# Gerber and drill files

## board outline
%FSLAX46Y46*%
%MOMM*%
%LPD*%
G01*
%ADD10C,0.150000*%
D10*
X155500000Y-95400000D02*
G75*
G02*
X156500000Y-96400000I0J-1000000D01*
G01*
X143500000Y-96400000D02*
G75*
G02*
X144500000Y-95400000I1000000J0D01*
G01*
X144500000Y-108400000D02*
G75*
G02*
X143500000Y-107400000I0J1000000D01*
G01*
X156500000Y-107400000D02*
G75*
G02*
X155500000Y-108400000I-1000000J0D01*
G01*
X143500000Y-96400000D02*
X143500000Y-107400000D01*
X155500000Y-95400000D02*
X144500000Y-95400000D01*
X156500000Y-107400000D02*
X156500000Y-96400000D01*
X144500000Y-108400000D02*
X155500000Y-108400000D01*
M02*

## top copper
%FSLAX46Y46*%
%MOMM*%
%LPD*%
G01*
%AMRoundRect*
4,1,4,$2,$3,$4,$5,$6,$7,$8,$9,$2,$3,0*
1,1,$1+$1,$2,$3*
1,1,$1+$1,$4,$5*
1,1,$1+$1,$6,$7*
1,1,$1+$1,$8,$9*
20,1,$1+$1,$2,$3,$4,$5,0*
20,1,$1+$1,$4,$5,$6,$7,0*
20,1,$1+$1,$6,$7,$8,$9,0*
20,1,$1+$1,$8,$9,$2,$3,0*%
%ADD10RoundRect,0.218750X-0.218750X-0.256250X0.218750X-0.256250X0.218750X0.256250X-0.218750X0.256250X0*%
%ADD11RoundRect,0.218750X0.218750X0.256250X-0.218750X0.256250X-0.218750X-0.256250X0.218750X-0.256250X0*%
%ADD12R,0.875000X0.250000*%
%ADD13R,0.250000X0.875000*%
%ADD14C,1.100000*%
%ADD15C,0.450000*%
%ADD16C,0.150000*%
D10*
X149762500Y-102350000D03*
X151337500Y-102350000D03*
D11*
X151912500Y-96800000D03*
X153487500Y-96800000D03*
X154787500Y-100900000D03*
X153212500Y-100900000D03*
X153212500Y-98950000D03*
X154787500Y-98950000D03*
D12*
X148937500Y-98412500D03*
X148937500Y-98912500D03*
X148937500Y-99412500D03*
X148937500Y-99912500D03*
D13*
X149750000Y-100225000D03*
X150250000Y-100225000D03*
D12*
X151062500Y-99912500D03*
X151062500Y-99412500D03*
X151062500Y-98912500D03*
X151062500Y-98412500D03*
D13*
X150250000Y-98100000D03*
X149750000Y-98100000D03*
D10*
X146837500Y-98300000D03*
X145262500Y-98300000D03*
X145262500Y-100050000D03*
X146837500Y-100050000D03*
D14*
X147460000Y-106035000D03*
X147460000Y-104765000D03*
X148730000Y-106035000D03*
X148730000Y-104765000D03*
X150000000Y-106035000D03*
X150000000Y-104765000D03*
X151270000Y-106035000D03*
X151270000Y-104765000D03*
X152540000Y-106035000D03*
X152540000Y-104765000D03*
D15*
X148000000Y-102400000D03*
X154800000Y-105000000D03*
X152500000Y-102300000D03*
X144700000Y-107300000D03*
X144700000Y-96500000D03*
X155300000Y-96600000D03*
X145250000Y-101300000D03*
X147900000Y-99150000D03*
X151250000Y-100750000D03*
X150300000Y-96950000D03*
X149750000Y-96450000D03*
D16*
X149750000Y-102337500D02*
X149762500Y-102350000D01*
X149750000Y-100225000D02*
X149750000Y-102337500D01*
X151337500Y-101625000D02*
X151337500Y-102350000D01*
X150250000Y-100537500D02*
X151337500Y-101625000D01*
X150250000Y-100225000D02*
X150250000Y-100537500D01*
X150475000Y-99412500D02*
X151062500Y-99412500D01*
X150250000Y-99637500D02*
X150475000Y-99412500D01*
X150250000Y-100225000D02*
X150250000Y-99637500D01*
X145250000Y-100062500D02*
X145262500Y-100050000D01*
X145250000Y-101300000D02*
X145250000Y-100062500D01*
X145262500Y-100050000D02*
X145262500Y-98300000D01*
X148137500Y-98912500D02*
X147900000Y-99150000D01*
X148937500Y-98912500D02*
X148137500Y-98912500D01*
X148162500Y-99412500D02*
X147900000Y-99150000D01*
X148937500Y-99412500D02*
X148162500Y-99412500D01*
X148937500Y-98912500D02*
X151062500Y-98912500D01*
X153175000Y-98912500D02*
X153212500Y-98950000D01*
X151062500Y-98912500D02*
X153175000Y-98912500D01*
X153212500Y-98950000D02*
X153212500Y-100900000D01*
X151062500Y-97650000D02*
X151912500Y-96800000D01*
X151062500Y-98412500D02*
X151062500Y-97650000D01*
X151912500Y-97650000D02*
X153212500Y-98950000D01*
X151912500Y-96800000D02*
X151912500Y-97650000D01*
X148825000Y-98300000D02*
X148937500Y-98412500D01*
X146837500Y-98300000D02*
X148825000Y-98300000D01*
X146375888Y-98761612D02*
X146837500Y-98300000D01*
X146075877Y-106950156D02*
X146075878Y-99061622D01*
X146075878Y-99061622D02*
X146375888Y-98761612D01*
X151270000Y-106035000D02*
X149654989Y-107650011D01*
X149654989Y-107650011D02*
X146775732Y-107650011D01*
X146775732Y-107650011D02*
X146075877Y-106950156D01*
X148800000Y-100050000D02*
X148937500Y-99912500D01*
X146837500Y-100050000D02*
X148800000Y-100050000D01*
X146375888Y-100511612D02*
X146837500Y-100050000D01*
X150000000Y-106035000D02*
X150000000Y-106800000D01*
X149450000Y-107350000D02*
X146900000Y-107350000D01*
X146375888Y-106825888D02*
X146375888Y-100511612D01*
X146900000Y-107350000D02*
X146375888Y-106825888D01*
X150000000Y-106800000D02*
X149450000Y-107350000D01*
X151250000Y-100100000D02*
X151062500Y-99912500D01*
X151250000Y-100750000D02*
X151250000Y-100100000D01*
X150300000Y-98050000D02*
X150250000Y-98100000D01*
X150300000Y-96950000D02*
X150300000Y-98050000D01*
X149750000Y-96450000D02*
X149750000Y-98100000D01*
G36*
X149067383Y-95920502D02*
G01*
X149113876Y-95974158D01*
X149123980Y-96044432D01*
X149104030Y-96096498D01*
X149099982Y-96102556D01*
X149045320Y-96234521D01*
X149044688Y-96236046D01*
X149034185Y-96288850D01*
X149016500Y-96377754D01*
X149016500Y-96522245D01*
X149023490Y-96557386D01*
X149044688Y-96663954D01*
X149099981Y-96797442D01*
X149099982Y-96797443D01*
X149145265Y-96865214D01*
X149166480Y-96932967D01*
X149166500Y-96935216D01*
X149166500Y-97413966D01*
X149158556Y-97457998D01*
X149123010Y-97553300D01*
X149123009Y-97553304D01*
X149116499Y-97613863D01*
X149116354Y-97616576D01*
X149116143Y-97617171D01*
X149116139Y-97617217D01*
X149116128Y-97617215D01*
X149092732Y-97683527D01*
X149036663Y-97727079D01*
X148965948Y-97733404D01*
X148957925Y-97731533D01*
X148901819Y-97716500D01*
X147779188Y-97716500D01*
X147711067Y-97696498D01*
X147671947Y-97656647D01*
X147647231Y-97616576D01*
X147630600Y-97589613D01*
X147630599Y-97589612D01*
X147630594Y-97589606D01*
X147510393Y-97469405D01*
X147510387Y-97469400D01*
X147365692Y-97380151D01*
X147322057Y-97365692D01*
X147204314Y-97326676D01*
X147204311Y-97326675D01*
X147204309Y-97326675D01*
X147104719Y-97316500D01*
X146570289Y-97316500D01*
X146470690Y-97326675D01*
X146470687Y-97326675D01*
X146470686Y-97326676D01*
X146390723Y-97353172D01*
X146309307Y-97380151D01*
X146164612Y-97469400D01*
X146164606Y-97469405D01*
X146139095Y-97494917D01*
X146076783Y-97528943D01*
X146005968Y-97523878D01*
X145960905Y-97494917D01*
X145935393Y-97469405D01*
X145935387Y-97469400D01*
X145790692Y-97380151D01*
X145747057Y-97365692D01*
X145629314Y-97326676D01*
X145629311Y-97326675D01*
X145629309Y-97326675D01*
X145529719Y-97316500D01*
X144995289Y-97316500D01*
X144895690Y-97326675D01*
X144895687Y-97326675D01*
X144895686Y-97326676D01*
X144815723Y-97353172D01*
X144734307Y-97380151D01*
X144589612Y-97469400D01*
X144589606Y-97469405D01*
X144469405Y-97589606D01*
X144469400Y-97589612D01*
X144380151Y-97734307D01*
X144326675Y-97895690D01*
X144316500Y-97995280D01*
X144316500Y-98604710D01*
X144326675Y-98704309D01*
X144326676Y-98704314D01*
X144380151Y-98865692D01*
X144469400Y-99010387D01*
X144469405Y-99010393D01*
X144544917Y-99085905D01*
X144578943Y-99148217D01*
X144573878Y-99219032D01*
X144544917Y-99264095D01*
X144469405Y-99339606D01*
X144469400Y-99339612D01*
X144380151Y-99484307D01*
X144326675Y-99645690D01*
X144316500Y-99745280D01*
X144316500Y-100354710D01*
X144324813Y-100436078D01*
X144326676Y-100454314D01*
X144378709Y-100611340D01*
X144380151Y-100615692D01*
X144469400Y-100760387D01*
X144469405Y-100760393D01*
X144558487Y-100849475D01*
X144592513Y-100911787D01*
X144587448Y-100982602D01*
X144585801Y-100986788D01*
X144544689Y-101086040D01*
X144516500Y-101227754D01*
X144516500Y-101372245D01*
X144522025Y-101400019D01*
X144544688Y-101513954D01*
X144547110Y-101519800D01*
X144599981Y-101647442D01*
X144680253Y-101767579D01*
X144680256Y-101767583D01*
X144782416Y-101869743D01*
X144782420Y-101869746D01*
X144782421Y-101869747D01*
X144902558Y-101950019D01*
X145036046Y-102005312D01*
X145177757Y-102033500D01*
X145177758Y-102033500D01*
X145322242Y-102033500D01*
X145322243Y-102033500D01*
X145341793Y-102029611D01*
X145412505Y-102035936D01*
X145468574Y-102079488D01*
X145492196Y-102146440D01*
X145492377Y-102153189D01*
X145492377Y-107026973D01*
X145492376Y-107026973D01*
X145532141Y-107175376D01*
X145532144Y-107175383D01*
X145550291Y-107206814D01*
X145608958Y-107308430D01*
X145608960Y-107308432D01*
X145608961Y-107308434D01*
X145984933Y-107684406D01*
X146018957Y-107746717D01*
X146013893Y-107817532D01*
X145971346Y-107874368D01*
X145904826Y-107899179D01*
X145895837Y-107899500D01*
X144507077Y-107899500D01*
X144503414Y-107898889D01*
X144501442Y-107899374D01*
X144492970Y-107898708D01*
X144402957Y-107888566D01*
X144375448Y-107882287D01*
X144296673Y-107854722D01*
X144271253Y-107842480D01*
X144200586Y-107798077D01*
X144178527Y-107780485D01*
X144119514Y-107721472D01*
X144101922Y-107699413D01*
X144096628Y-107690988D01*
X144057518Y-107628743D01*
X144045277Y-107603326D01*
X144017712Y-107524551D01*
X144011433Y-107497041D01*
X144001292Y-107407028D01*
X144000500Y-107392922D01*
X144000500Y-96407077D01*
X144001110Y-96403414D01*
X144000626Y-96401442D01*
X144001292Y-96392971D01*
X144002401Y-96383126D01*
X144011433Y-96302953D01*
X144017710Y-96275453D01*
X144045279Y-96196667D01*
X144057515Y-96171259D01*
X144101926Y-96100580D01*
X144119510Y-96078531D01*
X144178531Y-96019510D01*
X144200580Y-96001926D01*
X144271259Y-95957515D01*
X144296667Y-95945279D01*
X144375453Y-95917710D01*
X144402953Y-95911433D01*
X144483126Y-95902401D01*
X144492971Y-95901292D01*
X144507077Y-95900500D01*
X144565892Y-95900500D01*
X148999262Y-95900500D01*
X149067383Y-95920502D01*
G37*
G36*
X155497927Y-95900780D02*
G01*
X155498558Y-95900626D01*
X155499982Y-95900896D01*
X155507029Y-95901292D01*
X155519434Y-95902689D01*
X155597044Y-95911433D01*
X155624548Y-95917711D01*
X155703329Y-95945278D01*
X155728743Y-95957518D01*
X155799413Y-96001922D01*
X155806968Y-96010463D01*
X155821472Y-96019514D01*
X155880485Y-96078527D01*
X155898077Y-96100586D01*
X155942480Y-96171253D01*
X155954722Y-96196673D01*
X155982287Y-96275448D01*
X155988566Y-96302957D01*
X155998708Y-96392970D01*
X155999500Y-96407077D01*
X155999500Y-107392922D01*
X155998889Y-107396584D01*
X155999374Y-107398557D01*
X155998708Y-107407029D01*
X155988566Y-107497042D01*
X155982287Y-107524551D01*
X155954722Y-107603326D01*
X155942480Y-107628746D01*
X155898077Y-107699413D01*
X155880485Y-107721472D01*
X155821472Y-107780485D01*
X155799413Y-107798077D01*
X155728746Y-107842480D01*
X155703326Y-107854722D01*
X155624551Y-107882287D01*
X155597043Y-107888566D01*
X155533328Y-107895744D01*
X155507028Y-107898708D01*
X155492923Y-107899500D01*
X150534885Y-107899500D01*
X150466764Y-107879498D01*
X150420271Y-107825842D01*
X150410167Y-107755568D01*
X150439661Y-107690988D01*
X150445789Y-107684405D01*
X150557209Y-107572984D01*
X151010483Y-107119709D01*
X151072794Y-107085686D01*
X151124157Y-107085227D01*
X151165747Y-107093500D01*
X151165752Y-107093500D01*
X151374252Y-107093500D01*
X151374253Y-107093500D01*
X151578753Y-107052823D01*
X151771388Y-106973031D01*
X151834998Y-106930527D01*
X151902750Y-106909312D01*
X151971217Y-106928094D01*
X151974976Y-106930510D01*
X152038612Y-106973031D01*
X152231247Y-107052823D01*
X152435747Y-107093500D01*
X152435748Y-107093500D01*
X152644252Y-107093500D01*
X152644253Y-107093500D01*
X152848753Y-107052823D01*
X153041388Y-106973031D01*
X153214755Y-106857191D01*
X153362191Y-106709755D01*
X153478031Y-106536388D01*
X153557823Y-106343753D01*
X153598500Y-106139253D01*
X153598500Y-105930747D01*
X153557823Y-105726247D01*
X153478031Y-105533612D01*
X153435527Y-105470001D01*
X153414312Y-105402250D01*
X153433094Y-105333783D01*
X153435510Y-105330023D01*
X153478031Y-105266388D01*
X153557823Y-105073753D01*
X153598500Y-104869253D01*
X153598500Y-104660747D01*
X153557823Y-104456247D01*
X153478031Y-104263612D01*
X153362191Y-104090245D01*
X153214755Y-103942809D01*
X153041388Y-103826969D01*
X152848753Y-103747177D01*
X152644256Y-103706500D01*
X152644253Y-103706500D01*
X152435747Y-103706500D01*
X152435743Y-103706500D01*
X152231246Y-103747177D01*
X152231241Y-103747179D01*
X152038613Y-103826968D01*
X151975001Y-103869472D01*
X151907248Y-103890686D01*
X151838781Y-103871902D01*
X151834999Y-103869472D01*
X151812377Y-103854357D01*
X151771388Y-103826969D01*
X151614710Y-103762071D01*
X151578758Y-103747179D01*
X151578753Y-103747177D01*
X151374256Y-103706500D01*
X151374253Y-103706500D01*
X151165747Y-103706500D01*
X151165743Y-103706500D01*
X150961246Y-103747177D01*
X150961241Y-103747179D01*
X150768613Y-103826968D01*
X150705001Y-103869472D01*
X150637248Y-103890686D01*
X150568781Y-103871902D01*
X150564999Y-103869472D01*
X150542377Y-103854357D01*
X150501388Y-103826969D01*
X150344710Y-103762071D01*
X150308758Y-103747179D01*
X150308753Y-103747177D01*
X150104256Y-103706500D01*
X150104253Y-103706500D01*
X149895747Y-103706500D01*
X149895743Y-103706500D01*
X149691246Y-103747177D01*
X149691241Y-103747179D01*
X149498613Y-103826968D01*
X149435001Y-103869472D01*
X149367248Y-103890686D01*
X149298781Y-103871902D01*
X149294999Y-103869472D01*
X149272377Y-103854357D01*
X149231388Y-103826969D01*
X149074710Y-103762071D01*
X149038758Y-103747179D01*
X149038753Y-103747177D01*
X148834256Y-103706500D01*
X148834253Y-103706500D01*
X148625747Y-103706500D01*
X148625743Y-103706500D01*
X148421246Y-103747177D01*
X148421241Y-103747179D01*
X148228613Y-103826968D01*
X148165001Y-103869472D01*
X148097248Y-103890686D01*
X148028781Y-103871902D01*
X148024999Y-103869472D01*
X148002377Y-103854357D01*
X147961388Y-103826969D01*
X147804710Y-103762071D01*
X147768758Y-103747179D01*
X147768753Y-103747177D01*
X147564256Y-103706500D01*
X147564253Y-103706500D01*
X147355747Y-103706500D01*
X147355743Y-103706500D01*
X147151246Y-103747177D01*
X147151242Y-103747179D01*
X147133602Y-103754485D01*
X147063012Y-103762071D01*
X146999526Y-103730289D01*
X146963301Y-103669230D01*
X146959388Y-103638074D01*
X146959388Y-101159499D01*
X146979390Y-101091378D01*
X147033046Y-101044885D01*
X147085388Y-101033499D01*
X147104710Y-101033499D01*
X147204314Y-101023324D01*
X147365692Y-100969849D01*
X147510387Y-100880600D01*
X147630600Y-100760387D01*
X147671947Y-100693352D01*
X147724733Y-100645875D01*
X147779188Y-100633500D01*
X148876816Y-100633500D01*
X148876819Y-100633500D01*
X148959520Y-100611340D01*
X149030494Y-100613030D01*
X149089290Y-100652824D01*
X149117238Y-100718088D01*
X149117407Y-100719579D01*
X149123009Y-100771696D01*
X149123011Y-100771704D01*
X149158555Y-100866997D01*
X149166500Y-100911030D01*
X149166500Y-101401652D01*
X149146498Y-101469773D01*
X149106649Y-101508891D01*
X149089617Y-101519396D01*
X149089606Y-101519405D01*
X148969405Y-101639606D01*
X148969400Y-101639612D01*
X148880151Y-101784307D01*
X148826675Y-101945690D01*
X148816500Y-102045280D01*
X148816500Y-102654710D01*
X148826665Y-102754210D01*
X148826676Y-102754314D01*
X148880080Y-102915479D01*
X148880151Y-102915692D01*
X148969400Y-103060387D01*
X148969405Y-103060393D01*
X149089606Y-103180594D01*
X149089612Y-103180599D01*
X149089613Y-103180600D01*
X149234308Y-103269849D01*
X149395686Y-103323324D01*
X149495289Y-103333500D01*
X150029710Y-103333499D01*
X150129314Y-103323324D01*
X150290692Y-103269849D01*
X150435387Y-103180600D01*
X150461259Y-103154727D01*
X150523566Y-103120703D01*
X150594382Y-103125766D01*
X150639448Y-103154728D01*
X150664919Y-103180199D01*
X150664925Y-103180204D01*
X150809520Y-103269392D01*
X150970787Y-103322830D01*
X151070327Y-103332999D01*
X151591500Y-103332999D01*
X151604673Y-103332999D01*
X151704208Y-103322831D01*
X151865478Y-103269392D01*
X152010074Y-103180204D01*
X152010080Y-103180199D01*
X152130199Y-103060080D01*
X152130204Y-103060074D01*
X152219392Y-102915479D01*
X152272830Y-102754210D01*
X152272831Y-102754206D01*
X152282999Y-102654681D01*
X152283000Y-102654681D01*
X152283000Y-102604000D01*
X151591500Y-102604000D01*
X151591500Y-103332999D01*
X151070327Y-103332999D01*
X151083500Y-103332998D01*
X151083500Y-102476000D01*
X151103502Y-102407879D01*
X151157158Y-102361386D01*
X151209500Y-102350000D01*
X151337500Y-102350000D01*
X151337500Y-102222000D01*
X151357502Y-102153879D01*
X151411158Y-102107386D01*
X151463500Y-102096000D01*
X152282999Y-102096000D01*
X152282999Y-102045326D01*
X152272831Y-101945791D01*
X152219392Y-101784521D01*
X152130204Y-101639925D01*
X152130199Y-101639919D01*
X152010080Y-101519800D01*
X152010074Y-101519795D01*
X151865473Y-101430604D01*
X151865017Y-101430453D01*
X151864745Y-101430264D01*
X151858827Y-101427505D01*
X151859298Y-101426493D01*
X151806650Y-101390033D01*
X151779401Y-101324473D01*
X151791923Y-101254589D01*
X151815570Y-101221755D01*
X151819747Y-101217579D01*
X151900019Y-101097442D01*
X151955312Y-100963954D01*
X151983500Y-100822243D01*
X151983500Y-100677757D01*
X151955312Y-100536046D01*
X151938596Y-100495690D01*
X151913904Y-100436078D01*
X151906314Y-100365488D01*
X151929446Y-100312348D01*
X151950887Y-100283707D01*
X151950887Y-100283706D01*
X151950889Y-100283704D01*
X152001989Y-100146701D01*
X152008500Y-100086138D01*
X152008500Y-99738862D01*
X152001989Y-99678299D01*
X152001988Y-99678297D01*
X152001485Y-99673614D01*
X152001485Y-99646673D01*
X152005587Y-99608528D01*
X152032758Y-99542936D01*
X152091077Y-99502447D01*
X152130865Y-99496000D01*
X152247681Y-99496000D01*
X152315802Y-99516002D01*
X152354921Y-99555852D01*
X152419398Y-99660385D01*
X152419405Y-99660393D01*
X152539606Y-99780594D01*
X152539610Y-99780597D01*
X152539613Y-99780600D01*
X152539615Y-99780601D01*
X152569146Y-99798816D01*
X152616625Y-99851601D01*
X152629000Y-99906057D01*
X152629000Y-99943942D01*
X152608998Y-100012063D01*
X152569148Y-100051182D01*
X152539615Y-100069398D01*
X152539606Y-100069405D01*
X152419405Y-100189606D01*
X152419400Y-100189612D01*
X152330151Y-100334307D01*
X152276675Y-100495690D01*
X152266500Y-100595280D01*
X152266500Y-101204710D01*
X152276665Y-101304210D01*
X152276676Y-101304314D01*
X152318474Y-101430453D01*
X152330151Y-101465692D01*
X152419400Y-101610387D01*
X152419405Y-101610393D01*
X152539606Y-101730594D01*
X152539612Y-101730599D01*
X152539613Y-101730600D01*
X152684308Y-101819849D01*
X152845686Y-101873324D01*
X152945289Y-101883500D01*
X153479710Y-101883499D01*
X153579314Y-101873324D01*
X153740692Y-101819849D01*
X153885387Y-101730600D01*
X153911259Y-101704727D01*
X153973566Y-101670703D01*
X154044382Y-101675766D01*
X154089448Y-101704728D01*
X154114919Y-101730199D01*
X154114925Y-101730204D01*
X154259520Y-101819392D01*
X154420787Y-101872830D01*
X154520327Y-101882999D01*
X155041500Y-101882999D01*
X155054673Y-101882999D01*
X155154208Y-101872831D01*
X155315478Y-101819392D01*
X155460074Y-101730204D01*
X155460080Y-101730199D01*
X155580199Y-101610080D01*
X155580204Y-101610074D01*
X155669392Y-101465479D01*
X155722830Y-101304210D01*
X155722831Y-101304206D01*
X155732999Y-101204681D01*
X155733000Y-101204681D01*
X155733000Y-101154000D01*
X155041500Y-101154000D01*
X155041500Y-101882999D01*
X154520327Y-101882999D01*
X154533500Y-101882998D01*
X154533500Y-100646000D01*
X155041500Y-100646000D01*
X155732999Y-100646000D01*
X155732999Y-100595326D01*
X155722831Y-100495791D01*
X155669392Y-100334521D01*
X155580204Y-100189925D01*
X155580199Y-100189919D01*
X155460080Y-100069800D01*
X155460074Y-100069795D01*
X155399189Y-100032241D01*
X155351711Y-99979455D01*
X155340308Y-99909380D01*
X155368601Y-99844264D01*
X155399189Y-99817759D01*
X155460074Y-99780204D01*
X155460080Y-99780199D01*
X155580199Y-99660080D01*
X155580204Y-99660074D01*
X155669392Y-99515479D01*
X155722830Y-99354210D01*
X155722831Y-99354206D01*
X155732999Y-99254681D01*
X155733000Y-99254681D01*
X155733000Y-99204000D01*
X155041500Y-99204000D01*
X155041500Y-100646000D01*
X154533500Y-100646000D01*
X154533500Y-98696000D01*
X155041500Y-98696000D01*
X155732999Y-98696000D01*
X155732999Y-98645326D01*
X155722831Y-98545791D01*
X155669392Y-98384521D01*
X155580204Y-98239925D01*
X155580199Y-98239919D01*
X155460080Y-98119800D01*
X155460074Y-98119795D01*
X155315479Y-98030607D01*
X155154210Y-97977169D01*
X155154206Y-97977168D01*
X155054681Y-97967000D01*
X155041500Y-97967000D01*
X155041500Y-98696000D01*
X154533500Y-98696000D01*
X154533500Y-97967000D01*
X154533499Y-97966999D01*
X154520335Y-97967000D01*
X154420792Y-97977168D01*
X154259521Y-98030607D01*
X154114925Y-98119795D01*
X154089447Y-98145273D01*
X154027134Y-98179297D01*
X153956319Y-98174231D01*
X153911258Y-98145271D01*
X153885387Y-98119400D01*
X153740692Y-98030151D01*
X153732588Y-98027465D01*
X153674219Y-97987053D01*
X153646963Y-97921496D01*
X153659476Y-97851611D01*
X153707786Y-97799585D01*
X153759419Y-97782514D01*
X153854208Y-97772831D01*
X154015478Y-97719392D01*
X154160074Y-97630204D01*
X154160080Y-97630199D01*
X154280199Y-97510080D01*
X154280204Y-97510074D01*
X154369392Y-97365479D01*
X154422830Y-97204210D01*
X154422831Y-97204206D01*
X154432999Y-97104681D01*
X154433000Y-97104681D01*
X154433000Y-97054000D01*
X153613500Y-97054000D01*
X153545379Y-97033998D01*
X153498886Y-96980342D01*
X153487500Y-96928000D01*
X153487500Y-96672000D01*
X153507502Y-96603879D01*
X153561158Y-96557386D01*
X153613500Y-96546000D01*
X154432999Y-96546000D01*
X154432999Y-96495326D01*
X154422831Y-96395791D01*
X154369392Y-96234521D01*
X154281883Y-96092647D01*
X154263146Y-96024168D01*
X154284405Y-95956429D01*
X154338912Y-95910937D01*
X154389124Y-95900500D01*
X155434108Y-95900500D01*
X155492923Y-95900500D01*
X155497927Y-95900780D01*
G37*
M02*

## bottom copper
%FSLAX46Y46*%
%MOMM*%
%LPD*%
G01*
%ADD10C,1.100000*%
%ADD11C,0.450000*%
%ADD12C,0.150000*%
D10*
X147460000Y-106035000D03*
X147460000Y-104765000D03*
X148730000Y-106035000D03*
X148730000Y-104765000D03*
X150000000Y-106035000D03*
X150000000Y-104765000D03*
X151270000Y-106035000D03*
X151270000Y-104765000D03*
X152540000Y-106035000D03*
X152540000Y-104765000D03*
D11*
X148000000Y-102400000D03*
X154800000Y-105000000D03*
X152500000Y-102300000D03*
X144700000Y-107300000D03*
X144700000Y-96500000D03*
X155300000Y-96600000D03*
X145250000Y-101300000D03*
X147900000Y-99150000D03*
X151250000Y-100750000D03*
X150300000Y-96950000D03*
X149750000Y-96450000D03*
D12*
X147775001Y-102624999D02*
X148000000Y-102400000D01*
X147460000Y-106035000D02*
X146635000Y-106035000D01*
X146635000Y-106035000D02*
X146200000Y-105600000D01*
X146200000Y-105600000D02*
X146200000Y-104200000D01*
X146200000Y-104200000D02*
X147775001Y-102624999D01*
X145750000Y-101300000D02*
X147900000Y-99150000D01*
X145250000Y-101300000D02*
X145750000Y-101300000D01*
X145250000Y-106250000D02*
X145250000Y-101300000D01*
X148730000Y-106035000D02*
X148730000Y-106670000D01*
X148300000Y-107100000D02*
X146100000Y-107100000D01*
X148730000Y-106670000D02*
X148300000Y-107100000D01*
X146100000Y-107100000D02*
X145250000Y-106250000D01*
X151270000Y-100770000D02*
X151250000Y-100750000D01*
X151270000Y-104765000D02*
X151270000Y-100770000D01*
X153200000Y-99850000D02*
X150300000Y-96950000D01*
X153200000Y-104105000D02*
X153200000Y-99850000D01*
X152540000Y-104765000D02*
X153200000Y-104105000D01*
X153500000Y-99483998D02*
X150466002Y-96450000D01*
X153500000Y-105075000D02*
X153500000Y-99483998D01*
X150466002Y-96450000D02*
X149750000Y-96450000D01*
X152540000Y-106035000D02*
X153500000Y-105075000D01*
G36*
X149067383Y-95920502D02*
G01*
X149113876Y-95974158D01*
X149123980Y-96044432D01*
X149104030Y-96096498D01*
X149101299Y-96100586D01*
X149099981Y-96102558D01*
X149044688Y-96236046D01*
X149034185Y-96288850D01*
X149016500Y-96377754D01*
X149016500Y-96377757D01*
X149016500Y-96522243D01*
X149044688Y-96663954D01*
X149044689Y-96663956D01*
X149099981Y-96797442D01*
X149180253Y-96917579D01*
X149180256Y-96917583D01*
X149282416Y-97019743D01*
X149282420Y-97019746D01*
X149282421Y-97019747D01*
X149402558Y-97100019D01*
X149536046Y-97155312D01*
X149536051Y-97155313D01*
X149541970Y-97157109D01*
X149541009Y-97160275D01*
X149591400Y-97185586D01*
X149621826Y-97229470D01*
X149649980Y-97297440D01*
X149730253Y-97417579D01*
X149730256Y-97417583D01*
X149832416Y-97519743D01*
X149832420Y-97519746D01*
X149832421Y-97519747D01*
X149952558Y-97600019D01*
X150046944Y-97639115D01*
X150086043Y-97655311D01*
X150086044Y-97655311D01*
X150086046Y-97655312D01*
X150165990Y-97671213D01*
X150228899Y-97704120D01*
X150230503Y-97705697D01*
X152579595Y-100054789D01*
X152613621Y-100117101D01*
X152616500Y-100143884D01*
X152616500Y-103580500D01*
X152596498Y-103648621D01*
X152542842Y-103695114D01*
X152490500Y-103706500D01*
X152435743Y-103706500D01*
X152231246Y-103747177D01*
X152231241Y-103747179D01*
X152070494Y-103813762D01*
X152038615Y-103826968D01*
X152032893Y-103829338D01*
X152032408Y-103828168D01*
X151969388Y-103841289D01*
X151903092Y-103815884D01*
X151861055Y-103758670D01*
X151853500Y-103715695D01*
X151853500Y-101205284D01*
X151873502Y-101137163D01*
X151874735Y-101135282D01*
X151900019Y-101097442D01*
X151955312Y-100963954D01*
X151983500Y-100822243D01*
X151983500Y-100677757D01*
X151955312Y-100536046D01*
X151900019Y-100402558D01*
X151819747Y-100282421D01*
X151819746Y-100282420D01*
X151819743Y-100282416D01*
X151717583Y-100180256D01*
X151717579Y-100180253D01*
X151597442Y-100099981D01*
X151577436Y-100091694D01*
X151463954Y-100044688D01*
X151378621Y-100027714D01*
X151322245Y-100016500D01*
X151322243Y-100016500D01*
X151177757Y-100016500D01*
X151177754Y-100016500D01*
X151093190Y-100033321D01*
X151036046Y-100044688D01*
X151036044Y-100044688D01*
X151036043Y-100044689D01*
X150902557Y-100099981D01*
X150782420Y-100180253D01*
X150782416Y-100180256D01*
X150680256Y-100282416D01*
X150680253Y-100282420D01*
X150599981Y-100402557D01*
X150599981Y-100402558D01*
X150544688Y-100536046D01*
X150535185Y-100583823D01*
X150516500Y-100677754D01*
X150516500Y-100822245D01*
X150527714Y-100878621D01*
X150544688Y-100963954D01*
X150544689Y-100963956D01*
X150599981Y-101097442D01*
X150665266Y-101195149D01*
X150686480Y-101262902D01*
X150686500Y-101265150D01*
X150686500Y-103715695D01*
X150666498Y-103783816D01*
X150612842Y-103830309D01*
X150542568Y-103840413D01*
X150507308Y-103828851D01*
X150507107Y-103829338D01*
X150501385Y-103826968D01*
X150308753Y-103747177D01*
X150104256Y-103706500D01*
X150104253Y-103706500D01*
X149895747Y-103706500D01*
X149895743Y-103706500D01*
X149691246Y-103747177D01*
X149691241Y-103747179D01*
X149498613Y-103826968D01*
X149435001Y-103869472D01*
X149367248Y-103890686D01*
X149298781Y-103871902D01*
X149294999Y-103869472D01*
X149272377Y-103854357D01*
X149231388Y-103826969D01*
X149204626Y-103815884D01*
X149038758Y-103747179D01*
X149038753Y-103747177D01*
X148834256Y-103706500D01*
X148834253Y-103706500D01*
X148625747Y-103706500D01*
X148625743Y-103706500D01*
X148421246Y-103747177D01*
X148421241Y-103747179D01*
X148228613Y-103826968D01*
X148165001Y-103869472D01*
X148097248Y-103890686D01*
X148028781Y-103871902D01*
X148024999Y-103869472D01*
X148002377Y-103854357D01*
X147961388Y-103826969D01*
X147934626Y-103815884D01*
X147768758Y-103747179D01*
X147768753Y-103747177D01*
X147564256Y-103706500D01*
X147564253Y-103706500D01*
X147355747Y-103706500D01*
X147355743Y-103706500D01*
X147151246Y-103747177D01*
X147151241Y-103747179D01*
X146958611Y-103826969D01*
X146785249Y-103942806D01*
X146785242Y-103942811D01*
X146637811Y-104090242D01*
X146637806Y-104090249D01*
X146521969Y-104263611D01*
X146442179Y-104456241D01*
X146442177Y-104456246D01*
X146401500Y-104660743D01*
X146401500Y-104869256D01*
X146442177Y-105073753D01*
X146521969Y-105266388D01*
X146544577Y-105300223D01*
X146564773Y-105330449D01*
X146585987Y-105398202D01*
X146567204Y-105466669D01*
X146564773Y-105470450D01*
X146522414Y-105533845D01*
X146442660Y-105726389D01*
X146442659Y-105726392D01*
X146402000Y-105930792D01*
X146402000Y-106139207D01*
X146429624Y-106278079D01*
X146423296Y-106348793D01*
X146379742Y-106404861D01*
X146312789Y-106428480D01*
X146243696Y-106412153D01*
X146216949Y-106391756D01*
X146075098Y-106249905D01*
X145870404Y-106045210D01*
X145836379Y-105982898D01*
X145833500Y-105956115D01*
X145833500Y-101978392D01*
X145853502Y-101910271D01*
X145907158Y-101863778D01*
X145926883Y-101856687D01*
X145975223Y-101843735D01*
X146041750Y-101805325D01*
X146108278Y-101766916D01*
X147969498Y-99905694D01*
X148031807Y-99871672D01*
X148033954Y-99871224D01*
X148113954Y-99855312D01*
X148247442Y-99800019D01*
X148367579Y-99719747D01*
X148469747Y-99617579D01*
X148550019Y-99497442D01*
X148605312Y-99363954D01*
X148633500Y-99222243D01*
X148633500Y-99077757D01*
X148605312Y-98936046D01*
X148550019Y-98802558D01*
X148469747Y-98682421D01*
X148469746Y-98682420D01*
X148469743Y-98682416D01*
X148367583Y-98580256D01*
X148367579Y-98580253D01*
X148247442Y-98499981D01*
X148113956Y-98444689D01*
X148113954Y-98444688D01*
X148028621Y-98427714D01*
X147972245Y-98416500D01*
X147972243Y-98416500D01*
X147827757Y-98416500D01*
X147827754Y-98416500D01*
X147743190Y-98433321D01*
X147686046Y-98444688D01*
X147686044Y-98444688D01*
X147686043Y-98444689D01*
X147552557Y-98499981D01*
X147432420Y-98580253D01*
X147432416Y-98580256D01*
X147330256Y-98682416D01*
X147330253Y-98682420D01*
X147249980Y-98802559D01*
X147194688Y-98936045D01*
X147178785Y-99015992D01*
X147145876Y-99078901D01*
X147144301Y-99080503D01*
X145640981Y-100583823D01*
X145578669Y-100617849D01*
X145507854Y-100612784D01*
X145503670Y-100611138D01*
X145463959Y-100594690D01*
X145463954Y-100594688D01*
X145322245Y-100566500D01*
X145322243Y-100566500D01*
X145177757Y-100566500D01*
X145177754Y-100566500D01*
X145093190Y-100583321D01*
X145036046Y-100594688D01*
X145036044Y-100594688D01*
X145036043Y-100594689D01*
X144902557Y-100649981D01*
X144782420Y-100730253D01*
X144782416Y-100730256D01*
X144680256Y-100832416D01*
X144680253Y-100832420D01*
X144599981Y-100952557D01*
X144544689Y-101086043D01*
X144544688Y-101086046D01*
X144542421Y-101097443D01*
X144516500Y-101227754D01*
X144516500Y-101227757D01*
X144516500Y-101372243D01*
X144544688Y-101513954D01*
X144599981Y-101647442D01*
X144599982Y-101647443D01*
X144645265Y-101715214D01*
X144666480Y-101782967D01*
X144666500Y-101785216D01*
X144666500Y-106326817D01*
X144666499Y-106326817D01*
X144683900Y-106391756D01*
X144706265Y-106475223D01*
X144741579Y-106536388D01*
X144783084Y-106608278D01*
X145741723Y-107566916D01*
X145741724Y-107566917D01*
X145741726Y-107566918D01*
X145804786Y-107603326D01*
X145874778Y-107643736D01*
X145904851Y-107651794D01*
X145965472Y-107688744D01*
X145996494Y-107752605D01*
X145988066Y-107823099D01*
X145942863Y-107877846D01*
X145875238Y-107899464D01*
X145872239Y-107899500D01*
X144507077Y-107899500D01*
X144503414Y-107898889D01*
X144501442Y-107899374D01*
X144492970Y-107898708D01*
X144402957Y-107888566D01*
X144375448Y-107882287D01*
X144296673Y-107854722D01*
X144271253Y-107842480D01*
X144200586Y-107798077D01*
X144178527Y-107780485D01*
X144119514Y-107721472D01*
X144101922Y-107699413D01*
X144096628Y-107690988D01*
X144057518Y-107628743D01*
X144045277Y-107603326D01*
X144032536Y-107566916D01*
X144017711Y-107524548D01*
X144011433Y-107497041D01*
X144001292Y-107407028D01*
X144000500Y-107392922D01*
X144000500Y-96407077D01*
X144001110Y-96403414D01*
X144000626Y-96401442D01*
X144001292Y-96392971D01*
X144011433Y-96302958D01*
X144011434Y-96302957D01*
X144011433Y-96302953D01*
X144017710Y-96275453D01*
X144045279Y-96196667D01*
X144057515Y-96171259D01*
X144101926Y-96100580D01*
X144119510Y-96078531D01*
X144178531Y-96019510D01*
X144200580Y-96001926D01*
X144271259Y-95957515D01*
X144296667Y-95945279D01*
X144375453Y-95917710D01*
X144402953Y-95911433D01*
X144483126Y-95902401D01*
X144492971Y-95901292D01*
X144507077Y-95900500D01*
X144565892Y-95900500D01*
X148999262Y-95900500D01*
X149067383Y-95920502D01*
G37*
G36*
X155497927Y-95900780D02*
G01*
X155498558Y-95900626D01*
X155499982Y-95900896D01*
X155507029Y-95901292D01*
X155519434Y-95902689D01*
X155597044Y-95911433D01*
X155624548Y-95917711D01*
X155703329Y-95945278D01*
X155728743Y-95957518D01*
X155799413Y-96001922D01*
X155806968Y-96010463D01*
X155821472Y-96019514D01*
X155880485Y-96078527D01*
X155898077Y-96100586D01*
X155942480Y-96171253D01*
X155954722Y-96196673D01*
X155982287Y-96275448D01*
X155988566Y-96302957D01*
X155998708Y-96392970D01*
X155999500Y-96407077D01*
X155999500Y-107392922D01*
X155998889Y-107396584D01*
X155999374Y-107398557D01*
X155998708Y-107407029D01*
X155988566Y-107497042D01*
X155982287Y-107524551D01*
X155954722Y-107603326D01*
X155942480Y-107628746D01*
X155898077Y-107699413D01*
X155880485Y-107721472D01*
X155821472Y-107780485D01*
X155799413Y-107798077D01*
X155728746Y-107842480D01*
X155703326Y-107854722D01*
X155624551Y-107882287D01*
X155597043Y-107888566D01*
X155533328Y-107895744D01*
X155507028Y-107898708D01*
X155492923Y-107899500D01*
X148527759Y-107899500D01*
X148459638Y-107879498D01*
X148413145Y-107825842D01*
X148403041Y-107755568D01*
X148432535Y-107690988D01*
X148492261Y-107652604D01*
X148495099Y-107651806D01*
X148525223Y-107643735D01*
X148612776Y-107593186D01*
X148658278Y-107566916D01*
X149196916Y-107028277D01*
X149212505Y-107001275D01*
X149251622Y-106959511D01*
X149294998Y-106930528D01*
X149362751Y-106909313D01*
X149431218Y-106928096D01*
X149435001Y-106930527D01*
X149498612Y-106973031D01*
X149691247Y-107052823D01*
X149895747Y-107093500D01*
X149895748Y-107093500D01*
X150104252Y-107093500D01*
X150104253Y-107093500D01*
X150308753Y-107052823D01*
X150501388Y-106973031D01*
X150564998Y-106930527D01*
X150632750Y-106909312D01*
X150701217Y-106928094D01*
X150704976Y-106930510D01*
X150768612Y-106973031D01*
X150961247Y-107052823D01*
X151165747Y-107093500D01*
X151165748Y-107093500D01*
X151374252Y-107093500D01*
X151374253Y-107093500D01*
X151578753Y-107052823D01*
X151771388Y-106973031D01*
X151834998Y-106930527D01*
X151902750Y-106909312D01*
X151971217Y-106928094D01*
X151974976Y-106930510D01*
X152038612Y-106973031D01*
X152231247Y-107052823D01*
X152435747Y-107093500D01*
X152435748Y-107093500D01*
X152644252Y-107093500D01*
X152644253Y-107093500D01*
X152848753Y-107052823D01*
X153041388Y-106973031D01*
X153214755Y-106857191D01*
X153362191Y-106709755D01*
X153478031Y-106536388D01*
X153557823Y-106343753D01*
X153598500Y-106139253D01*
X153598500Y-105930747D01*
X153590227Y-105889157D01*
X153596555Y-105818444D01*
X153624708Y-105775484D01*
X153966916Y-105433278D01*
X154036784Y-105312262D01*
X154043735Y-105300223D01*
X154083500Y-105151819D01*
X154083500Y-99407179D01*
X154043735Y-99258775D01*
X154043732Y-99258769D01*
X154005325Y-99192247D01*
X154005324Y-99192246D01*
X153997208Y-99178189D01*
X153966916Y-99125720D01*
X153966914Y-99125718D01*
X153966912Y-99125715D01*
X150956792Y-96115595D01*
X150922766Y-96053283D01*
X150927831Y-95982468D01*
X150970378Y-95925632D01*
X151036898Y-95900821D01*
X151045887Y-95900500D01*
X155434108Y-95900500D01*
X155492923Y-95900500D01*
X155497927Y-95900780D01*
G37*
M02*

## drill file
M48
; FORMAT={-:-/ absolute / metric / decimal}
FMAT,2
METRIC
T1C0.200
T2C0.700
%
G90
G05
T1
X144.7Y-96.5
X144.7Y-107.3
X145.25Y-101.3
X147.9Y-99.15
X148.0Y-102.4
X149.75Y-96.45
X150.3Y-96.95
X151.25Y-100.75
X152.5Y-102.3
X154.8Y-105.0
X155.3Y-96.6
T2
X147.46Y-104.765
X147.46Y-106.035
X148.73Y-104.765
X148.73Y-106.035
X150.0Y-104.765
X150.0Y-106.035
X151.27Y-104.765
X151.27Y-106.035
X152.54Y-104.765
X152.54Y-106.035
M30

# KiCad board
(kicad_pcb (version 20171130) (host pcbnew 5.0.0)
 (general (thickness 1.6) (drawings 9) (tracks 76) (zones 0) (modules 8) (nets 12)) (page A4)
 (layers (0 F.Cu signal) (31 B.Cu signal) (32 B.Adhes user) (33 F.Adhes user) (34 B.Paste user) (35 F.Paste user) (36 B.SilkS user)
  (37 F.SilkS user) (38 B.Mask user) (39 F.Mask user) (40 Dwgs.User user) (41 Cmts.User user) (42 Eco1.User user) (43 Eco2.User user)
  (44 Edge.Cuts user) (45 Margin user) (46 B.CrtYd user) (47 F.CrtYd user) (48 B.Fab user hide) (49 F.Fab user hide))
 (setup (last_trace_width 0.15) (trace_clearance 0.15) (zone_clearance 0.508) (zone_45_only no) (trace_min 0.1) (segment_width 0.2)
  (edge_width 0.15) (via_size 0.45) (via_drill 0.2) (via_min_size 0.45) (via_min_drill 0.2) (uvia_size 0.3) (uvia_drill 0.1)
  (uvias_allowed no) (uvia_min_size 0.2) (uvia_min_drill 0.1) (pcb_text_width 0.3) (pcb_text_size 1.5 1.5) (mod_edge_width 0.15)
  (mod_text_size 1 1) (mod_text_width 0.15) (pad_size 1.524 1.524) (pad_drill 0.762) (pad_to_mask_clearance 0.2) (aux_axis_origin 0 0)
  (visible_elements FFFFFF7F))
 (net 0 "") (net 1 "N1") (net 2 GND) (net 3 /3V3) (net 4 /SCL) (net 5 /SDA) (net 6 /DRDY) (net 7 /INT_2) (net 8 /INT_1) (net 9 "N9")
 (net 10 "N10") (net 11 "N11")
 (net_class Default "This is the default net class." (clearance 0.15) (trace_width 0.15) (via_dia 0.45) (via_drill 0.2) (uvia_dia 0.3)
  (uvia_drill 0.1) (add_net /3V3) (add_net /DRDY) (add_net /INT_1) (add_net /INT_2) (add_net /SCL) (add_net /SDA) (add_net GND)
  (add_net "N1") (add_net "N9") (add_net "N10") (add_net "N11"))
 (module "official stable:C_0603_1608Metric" (layer F.Cu) (at 150.55 102.35)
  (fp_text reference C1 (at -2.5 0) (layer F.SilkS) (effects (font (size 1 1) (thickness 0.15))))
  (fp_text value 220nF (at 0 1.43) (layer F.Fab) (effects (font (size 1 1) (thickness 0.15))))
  (pad 1 smd roundrect (at -0.7875 0) (size 0.875 0.95) (layers F.Cu F.Paste F.Mask) (roundrect_rratio 0.25) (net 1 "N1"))
  (pad 2 smd roundrect (at 0.7875 0) (size 0.875 0.95) (layers F.Cu F.Paste F.Mask) (roundrect_rratio 0.25) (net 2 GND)))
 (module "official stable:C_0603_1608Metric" (layer F.Cu) (at 152.7 96.8 180)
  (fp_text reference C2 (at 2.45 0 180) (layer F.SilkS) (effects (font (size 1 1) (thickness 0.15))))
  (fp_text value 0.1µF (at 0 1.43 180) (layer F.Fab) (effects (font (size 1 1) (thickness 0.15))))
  (pad 2 smd roundrect (at 0.7875 0 180) (size 0.875 0.95) (layers F.Cu F.Paste F.Mask) (roundrect_rratio 0.25) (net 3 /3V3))
  (pad 1 smd roundrect (at -0.7875 0 180) (size 0.875 0.95) (layers F.Cu F.Paste F.Mask) (roundrect_rratio 0.25) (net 2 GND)))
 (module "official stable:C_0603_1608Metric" (layer F.Cu) (at 154 100.9 180)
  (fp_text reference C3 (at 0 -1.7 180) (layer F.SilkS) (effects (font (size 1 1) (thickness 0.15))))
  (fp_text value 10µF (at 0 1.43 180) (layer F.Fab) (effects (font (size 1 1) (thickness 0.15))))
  (pad 1 smd roundrect (at -0.7875 0 180) (size 0.875 0.95) (layers F.Cu F.Paste F.Mask) (roundrect_rratio 0.25) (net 2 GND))
  (pad 2 smd roundrect (at 0.7875 0 180) (size 0.875 0.95) (layers F.Cu F.Paste F.Mask) (roundrect_rratio 0.25) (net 3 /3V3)))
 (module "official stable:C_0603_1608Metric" (layer F.Cu) (at 154 98.95 180)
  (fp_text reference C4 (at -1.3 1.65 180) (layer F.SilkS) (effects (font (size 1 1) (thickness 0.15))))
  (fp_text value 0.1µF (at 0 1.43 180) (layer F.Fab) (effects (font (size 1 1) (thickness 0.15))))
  (pad 2 smd roundrect (at 0.7875 0 180) (size 0.875 0.95) (layers F.Cu F.Paste F.Mask) (roundrect_rratio 0.25) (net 3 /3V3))
  (pad 1 smd roundrect (at -0.7875 0 180) (size 0.875 0.95) (layers F.Cu F.Paste F.Mask) (roundrect_rratio 0.25) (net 2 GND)))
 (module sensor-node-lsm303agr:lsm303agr (layer F.Cu) (at 150 99.1625)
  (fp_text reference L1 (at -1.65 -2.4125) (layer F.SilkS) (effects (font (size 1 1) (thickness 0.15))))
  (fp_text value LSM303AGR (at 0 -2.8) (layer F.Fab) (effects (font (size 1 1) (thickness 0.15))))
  (pad 1 smd rect (at -1.0625 -0.75) (size 0.875 0.25) (layers F.Cu F.Paste F.Mask) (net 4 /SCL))
  (pad 2 smd rect (at -1.0625 -0.25) (size 0.875 0.25) (layers F.Cu F.Paste F.Mask) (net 3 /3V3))
  (pad 3 smd rect (at -1.0625 0.25) (size 0.875 0.25) (layers F.Cu F.Paste F.Mask) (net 3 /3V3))
  (pad 4 smd rect (at -1.0625 0.75) (size 0.875 0.25) (layers F.Cu F.Paste F.Mask) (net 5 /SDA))
  (pad 5 smd rect (at -0.25 1.0625) (size 0.25 0.875) (layers F.Cu F.Paste F.Mask) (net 1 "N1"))
  (pad 6 smd rect (at 0.25 1.0625) (size 0.25 0.875) (layers F.Cu F.Paste F.Mask) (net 2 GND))
  (pad 7 smd rect (at 1.0625 0.75) (size 0.875 0.25) (layers F.Cu F.Paste F.Mask) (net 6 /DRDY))
  (pad 8 smd rect (at 1.0625 0.25) (size 0.875 0.25) (layers F.Cu F.Paste F.Mask) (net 2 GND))
  (pad 9 smd rect (at 1.0625 -0.25) (size 0.875 0.25) (layers F.Cu F.Paste F.Mask) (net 3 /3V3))
  (pad 10 smd rect (at 1.0625 -0.75) (size 0.875 0.25) (layers F.Cu F.Paste F.Mask) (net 3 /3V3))
  (pad 11 smd rect (at 0.25 -1.0625) (size 0.25 0.875) (layers F.Cu F.Paste F.Mask) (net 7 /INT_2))
  (pad 12 smd rect (at -0.25 -1.0625) (size 0.25 0.875) (layers F.Cu F.Paste F.Mask) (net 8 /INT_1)))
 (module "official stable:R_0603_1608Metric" (layer F.Cu) (at 146.05 98.3)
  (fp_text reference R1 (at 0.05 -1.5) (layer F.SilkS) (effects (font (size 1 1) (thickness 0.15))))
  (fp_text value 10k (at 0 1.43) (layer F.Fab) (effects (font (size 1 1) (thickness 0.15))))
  (pad 2 smd roundrect (at 0.7875 0) (size 0.875 0.95) (layers F.Cu F.Paste F.Mask) (roundrect_rratio 0.25) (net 4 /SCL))
  (pad 1 smd roundrect (at -0.7875 0) (size 0.875 0.95) (layers F.Cu F.Paste F.Mask) (roundrect_rratio 0.25) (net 3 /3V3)))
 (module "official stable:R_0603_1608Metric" (layer F.Cu) (at 146.05 100.05)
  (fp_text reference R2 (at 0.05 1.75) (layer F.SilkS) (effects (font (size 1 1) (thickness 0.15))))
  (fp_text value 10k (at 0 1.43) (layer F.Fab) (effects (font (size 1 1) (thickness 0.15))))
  (pad 1 smd roundrect (at -0.7875 0) (size 0.875 0.95) (layers F.Cu F.Paste F.Mask) (roundrect_rratio 0.25) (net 3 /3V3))
  (pad 2 smd roundrect (at 0.7875 0) (size 0.875 0.95) (layers F.Cu F.Paste F.Mask) (roundrect_rratio 0.25) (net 5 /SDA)))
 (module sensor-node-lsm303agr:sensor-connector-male (layer F.Cu) (at 150 105.4)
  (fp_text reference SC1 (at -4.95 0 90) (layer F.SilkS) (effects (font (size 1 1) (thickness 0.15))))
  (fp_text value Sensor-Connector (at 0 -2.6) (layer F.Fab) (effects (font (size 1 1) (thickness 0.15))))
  (pad 1 thru_hole circle (at -2.54 0.635) (size 1.1 1.1) (drill 0.7) (layers *.Cu *.Mask) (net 2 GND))
  (pad 2 thru_hole circle (at -2.54 -0.635) (size 1.1 1.1) (drill 0.7) (layers *.Cu *.Mask) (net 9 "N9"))
  (pad 3 thru_hole circle (at -1.27 0.635) (size 1.1 1.1) (drill 0.7) (layers *.Cu *.Mask) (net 3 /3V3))
  (pad 4 thru_hole circle (at -1.27 -0.635) (size 1.1 1.1) (drill 0.7) (layers *.Cu *.Mask) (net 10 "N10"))
  (pad 5 thru_hole circle (at 0 0.635) (size 1.1 1.1) (drill 0.7) (layers *.Cu *.Mask) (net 5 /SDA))
  (pad 6 thru_hole circle (at 0 -0.635) (size 1.1 1.1) (drill 0.7) (layers *.Cu *.Mask) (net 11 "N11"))
  (pad 7 thru_hole circle (at 1.27 0.635) (size 1.1 1.1) (drill 0.7) (layers *.Cu *.Mask) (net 4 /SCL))
  (pad 8 thru_hole circle (at 1.27 -0.635) (size 1.1 1.1) (drill 0.7) (layers *.Cu *.Mask) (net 6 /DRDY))
  (pad 9 thru_hole circle (at 2.54 0.635) (size 1.1 1.1) (drill 0.7) (layers *.Cu *.Mask) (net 8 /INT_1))
  (pad 10 thru_hole circle (at 2.54 -0.635) (size 1.1 1.1) (drill 0.7) (layers *.Cu *.Mask) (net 7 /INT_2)))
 (gr_arc (start 155.5 96.4) (end 156.5 96.4) (angle -90) (layer Edge.Cuts) (width 0.15))
 (gr_arc (start 144.5 96.4) (end 144.5 95.4) (angle -90) (layer Edge.Cuts) (width 0.15))
 (gr_arc (start 144.5 107.4) (end 143.5 107.4) (angle -90) (layer Edge.Cuts) (width 0.15))
 (gr_arc (start 155.5 107.4) (end 155.5 108.4) (angle -90) (layer Edge.Cuts) (width 0.15))
 (gr_line (start 143.5 96.4) (end 143.5 107.4) (layer Edge.Cuts) (width 0.15))
 (gr_line (start 155.5 95.4) (end 144.5 95.4) (layer Edge.Cuts) (width 0.15))
 (gr_line (start 156.5 107.4) (end 156.5 96.4) (layer Edge.Cuts) (width 0.15))
 (gr_line (start 144.5 108.4) (end 155.5 108.4) (layer Edge.Cuts) (width 0.15))
 (segment (start 149.75 102.3375) (end 149.7625 102.35) (width 0.15) (layer F.Cu) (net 1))
 (segment (start 149.75 100.225) (end 149.75 102.3375) (width 0.15) (layer F.Cu) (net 1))
 (via (at 148 102.4) (size 0.45) (drill 0.2) (layers F.Cu B.Cu) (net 2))
 (via (at 154.8 105) (size 0.45) (drill 0.2) (layers F.Cu B.Cu) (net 2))
 (via (at 152.5 102.3) (size 0.45) (drill 0.2) (layers F.Cu B.Cu) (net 2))
 (segment (start 147.775001 102.624999) (end 148 102.4) (width 0.15) (layer B.Cu) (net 2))
 (segment (start 147.46 106.035) (end 146.635 106.035) (width 0.15) (layer B.Cu) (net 2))
 (segment (start 146.635 106.035) (end 146.2 105.6) (width 0.15) (layer B.Cu) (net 2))
 (segment (start 146.2 105.6) (end 146.2 104.2) (width 0.15) (layer B.Cu) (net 2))
 (segment (start 146.2 104.2) (end 147.775001 102.624999) (width 0.15) (layer B.Cu) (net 2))
 (via (at 144.7 107.3) (size 0.45) (drill 0.2) (layers F.Cu B.Cu) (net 2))
 (via (at 144.7 96.5) (size 0.45) (drill 0.2) (layers F.Cu B.Cu) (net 2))
 (via (at 155.3 96.6) (size 0.45) (drill 0.2) (layers F.Cu B.Cu) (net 2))
 (segment (start 151.3375 101.625) (end 151.3375 102.35) (width 0.15) (layer F.Cu) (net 2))
 (segment (start 150.25 100.5375) (end 151.3375 101.625) (width 0.15) (layer F.Cu) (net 2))
 (segment (start 150.25 100.225) (end 150.25 100.5375) (width 0.15) (layer F.Cu) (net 2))
 (segment (start 150.475 99.4125) (end 151.0625 99.4125) (width 0.15) (layer F.Cu) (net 2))
 (segment (start 150.25 99.6375) (end 150.475 99.4125) (width 0.15) (layer F.Cu) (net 2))
 (segment (start 150.25 100.225) (end 150.25 99.6375) (width 0.15) (layer F.Cu) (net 2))
 (via (at 145.25 101.3) (size 0.45) (drill 0.2) (layers F.Cu B.Cu) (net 3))
 (segment (start 145.25 100.0625) (end 145.2625 100.05) (width 0.15) (layer F.Cu) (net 3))
 (segment (start 145.25 101.3) (end 145.25 100.0625) (width 0.15) (layer F.Cu) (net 3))
 (segment (start 145.2625 100.05) (end 145.2625 98.3) (width 0.15) (layer F.Cu) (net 3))
 (via (at 147.9 99.15) (size 0.45) (drill 0.2) (layers F.Cu B.Cu) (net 3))
 (segment (start 145.75 101.3) (end 147.9 99.15) (width 0.15) (layer B.Cu) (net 3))
 (segment (start 145.25 101.3) (end 145.75 101.3) (width 0.15) (layer B.Cu) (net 3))
 (segment (start 148.1375 98.9125) (end 147.9 99.15) (width 0.15) (layer F.Cu) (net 3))
 (segment (start 148.9375 98.9125) (end 148.1375 98.9125) (width 0.15) (layer F.Cu) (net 3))
 (segment (start 148.1625 99.4125) (end 147.9 99.15) (width 0.15) (layer F.Cu) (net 3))
 (segment (start 148.9375 99.4125) (end 148.1625 99.4125) (width 0.15) (layer F.Cu) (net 3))
 (segment (start 148.9375 98.9125) (end 151.0625 98.9125) (width 0.15) (layer F.Cu) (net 3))
 (segment (start 153.175 98.9125) (end 153.2125 98.95) (width 0.15) (layer F.Cu) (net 3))
 (segment (start 151.0625 98.9125) (end 153.175 98.9125) (width 0.15) (layer F.Cu) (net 3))
 (segment (start 153.2125 98.95) (end 153.2125 100.9) (width 0.15) (layer F.Cu) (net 3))
 (segment (start 151.0625 97.65) (end 151.9125 96.8) (width 0.15) (layer F.Cu) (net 3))
 (segment (start 151.0625 98.4125) (end 151.0625 97.65) (width 0.15) (layer F.Cu) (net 3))
 (segment (start 151.9125 97.65) (end 153.2125 98.95) (width 0.15) (layer F.Cu) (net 3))
 (segment (start 151.9125 96.8) (end 151.9125 97.65) (width 0.15) (layer F.Cu) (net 3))
 (segment (start 145.25 106.25) (end 145.25 101.3) (width 0.15) (layer B.Cu) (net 3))
 (segment (start 148.73 106.035) (end 148.73 106.67) (width 0.15) (layer B.Cu) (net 3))
 (segment (start 148.3 107.1) (end 146.1 107.1) (width 0.15) (layer B.Cu) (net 3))
 (segment (start 148.73 106.67) (end 148.3 107.1) (width 0.15) (layer B.Cu) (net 3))
 (segment (start 146.1 107.1) (end 145.25 106.25) (width 0.15) (layer B.Cu) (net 3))
 (segment (start 148.825 98.3) (end 148.9375 98.4125) (width 0.15) (layer F.Cu) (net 4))
 (segment (start 146.8375 98.3) (end 148.825 98.3) (width 0.15) (layer F.Cu) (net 4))
 (segment (start 146.375888 98.761612) (end 146.8375 98.3) (width 0.15) (layer F.Cu) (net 4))
 (segment (start 146.075877 106.950156) (end 146.075878 99.061622) (width 0.15) (layer F.Cu) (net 4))
 (segment (start 146.075878 99.061622) (end 146.375888 98.761612) (width 0.15) (layer F.Cu) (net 4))
 (segment (start 151.27 106.035) (end 149.654989 107.650011) (width 0.15) (layer F.Cu) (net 4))
 (segment (start 149.654989 107.650011) (end 146.775732 107.650011) (width 0.15) (layer F.Cu) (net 4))
 (segment (start 146.775732 107.650011) (end 146.075877 106.950156) (width 0.15) (layer F.Cu) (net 4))
 (segment (start 148.8 100.05) (end 148.9375 99.9125) (width 0.15) (layer F.Cu) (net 5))
 (segment (start 146.8375 100.05) (end 148.8 100.05) (width 0.15) (layer F.Cu) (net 5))
 (segment (start 146.375888 100.511612) (end 146.8375 100.05) (width 0.15) (layer F.Cu) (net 5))
 (segment (start 150 106.035) (end 150 106.8) (width 0.15) (layer F.Cu) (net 5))
 (segment (start 149.45 107.35) (end 146.9 107.35) (width 0.15) (layer F.Cu) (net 5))
 (segment (start 146.375888 106.825888) (end 146.375888 100.511612) (width 0.15) (layer F.Cu) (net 5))
 (segment (start 146.9 107.35) (end 146.375888 106.825888) (width 0.15) (layer F.Cu) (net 5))
 (segment (start 150 106.8) (end 149.45 107.35) (width 0.15) (layer F.Cu) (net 5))
 (via (at 151.25 100.75) (size 0.45) (drill 0.2) (layers F.Cu B.Cu) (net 6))
 (segment (start 151.27 100.77) (end 151.25 100.75) (width 0.15) (layer B.Cu) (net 6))
 (segment (start 151.27 104.765) (end 151.27 100.77) (width 0.15) (layer B.Cu) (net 6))
 (segment (start 151.25 100.1) (end 151.0625 99.9125) (width 0.15) (layer F.Cu) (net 6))
 (segment (start 151.25 100.75) (end 151.25 100.1) (width 0.15) (layer F.Cu) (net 6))
 (via (at 150.3 96.95) (size 0.45) (drill 0.2) (layers F.Cu B.Cu) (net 7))
 (segment (start 150.3 98.05) (end 150.25 98.1) (width 0.15) (layer F.Cu) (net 7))
 (segment (start 150.3 96.95) (end 150.3 98.05) (width 0.15) (layer F.Cu) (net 7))
 (segment (start 153.2 99.85) (end 150.3 96.95) (width 0.15) (layer B.Cu) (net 7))
 (segment (start 153.2 104.105) (end 153.2 99.85) (width 0.15) (layer B.Cu) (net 7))
 (segment (start 152.54 104.765) (end 153.2 104.105) (width 0.15) (layer B.Cu) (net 7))
 (via (at 149.75 96.45) (size 0.45) (drill 0.2) (layers F.Cu B.Cu) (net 8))
 (segment (start 149.75 96.45) (end 149.75 98.1) (width 0.15) (layer F.Cu) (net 8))
 (segment (start 153.5 99.483998) (end 150.466002 96.45) (width 0.15) (layer B.Cu) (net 8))
 (segment (start 153.5 105.075) (end 153.5 99.483998) (width 0.15) (layer B.Cu) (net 8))
 (segment (start 150.466002 96.45) (end 149.75 96.45) (width 0.15) (layer B.Cu) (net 8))
 (segment (start 152.54 106.035) (end 153.5 105.075) (width 0.15) (layer B.Cu) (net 8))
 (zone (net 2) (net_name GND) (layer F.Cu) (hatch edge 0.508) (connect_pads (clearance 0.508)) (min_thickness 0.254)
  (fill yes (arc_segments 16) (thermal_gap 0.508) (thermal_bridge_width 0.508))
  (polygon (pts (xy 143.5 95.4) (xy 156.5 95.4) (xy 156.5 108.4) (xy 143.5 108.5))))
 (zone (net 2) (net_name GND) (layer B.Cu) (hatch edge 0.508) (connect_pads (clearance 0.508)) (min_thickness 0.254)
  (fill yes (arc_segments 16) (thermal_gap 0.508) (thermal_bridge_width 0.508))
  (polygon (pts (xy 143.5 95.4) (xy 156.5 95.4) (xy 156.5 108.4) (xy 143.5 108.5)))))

